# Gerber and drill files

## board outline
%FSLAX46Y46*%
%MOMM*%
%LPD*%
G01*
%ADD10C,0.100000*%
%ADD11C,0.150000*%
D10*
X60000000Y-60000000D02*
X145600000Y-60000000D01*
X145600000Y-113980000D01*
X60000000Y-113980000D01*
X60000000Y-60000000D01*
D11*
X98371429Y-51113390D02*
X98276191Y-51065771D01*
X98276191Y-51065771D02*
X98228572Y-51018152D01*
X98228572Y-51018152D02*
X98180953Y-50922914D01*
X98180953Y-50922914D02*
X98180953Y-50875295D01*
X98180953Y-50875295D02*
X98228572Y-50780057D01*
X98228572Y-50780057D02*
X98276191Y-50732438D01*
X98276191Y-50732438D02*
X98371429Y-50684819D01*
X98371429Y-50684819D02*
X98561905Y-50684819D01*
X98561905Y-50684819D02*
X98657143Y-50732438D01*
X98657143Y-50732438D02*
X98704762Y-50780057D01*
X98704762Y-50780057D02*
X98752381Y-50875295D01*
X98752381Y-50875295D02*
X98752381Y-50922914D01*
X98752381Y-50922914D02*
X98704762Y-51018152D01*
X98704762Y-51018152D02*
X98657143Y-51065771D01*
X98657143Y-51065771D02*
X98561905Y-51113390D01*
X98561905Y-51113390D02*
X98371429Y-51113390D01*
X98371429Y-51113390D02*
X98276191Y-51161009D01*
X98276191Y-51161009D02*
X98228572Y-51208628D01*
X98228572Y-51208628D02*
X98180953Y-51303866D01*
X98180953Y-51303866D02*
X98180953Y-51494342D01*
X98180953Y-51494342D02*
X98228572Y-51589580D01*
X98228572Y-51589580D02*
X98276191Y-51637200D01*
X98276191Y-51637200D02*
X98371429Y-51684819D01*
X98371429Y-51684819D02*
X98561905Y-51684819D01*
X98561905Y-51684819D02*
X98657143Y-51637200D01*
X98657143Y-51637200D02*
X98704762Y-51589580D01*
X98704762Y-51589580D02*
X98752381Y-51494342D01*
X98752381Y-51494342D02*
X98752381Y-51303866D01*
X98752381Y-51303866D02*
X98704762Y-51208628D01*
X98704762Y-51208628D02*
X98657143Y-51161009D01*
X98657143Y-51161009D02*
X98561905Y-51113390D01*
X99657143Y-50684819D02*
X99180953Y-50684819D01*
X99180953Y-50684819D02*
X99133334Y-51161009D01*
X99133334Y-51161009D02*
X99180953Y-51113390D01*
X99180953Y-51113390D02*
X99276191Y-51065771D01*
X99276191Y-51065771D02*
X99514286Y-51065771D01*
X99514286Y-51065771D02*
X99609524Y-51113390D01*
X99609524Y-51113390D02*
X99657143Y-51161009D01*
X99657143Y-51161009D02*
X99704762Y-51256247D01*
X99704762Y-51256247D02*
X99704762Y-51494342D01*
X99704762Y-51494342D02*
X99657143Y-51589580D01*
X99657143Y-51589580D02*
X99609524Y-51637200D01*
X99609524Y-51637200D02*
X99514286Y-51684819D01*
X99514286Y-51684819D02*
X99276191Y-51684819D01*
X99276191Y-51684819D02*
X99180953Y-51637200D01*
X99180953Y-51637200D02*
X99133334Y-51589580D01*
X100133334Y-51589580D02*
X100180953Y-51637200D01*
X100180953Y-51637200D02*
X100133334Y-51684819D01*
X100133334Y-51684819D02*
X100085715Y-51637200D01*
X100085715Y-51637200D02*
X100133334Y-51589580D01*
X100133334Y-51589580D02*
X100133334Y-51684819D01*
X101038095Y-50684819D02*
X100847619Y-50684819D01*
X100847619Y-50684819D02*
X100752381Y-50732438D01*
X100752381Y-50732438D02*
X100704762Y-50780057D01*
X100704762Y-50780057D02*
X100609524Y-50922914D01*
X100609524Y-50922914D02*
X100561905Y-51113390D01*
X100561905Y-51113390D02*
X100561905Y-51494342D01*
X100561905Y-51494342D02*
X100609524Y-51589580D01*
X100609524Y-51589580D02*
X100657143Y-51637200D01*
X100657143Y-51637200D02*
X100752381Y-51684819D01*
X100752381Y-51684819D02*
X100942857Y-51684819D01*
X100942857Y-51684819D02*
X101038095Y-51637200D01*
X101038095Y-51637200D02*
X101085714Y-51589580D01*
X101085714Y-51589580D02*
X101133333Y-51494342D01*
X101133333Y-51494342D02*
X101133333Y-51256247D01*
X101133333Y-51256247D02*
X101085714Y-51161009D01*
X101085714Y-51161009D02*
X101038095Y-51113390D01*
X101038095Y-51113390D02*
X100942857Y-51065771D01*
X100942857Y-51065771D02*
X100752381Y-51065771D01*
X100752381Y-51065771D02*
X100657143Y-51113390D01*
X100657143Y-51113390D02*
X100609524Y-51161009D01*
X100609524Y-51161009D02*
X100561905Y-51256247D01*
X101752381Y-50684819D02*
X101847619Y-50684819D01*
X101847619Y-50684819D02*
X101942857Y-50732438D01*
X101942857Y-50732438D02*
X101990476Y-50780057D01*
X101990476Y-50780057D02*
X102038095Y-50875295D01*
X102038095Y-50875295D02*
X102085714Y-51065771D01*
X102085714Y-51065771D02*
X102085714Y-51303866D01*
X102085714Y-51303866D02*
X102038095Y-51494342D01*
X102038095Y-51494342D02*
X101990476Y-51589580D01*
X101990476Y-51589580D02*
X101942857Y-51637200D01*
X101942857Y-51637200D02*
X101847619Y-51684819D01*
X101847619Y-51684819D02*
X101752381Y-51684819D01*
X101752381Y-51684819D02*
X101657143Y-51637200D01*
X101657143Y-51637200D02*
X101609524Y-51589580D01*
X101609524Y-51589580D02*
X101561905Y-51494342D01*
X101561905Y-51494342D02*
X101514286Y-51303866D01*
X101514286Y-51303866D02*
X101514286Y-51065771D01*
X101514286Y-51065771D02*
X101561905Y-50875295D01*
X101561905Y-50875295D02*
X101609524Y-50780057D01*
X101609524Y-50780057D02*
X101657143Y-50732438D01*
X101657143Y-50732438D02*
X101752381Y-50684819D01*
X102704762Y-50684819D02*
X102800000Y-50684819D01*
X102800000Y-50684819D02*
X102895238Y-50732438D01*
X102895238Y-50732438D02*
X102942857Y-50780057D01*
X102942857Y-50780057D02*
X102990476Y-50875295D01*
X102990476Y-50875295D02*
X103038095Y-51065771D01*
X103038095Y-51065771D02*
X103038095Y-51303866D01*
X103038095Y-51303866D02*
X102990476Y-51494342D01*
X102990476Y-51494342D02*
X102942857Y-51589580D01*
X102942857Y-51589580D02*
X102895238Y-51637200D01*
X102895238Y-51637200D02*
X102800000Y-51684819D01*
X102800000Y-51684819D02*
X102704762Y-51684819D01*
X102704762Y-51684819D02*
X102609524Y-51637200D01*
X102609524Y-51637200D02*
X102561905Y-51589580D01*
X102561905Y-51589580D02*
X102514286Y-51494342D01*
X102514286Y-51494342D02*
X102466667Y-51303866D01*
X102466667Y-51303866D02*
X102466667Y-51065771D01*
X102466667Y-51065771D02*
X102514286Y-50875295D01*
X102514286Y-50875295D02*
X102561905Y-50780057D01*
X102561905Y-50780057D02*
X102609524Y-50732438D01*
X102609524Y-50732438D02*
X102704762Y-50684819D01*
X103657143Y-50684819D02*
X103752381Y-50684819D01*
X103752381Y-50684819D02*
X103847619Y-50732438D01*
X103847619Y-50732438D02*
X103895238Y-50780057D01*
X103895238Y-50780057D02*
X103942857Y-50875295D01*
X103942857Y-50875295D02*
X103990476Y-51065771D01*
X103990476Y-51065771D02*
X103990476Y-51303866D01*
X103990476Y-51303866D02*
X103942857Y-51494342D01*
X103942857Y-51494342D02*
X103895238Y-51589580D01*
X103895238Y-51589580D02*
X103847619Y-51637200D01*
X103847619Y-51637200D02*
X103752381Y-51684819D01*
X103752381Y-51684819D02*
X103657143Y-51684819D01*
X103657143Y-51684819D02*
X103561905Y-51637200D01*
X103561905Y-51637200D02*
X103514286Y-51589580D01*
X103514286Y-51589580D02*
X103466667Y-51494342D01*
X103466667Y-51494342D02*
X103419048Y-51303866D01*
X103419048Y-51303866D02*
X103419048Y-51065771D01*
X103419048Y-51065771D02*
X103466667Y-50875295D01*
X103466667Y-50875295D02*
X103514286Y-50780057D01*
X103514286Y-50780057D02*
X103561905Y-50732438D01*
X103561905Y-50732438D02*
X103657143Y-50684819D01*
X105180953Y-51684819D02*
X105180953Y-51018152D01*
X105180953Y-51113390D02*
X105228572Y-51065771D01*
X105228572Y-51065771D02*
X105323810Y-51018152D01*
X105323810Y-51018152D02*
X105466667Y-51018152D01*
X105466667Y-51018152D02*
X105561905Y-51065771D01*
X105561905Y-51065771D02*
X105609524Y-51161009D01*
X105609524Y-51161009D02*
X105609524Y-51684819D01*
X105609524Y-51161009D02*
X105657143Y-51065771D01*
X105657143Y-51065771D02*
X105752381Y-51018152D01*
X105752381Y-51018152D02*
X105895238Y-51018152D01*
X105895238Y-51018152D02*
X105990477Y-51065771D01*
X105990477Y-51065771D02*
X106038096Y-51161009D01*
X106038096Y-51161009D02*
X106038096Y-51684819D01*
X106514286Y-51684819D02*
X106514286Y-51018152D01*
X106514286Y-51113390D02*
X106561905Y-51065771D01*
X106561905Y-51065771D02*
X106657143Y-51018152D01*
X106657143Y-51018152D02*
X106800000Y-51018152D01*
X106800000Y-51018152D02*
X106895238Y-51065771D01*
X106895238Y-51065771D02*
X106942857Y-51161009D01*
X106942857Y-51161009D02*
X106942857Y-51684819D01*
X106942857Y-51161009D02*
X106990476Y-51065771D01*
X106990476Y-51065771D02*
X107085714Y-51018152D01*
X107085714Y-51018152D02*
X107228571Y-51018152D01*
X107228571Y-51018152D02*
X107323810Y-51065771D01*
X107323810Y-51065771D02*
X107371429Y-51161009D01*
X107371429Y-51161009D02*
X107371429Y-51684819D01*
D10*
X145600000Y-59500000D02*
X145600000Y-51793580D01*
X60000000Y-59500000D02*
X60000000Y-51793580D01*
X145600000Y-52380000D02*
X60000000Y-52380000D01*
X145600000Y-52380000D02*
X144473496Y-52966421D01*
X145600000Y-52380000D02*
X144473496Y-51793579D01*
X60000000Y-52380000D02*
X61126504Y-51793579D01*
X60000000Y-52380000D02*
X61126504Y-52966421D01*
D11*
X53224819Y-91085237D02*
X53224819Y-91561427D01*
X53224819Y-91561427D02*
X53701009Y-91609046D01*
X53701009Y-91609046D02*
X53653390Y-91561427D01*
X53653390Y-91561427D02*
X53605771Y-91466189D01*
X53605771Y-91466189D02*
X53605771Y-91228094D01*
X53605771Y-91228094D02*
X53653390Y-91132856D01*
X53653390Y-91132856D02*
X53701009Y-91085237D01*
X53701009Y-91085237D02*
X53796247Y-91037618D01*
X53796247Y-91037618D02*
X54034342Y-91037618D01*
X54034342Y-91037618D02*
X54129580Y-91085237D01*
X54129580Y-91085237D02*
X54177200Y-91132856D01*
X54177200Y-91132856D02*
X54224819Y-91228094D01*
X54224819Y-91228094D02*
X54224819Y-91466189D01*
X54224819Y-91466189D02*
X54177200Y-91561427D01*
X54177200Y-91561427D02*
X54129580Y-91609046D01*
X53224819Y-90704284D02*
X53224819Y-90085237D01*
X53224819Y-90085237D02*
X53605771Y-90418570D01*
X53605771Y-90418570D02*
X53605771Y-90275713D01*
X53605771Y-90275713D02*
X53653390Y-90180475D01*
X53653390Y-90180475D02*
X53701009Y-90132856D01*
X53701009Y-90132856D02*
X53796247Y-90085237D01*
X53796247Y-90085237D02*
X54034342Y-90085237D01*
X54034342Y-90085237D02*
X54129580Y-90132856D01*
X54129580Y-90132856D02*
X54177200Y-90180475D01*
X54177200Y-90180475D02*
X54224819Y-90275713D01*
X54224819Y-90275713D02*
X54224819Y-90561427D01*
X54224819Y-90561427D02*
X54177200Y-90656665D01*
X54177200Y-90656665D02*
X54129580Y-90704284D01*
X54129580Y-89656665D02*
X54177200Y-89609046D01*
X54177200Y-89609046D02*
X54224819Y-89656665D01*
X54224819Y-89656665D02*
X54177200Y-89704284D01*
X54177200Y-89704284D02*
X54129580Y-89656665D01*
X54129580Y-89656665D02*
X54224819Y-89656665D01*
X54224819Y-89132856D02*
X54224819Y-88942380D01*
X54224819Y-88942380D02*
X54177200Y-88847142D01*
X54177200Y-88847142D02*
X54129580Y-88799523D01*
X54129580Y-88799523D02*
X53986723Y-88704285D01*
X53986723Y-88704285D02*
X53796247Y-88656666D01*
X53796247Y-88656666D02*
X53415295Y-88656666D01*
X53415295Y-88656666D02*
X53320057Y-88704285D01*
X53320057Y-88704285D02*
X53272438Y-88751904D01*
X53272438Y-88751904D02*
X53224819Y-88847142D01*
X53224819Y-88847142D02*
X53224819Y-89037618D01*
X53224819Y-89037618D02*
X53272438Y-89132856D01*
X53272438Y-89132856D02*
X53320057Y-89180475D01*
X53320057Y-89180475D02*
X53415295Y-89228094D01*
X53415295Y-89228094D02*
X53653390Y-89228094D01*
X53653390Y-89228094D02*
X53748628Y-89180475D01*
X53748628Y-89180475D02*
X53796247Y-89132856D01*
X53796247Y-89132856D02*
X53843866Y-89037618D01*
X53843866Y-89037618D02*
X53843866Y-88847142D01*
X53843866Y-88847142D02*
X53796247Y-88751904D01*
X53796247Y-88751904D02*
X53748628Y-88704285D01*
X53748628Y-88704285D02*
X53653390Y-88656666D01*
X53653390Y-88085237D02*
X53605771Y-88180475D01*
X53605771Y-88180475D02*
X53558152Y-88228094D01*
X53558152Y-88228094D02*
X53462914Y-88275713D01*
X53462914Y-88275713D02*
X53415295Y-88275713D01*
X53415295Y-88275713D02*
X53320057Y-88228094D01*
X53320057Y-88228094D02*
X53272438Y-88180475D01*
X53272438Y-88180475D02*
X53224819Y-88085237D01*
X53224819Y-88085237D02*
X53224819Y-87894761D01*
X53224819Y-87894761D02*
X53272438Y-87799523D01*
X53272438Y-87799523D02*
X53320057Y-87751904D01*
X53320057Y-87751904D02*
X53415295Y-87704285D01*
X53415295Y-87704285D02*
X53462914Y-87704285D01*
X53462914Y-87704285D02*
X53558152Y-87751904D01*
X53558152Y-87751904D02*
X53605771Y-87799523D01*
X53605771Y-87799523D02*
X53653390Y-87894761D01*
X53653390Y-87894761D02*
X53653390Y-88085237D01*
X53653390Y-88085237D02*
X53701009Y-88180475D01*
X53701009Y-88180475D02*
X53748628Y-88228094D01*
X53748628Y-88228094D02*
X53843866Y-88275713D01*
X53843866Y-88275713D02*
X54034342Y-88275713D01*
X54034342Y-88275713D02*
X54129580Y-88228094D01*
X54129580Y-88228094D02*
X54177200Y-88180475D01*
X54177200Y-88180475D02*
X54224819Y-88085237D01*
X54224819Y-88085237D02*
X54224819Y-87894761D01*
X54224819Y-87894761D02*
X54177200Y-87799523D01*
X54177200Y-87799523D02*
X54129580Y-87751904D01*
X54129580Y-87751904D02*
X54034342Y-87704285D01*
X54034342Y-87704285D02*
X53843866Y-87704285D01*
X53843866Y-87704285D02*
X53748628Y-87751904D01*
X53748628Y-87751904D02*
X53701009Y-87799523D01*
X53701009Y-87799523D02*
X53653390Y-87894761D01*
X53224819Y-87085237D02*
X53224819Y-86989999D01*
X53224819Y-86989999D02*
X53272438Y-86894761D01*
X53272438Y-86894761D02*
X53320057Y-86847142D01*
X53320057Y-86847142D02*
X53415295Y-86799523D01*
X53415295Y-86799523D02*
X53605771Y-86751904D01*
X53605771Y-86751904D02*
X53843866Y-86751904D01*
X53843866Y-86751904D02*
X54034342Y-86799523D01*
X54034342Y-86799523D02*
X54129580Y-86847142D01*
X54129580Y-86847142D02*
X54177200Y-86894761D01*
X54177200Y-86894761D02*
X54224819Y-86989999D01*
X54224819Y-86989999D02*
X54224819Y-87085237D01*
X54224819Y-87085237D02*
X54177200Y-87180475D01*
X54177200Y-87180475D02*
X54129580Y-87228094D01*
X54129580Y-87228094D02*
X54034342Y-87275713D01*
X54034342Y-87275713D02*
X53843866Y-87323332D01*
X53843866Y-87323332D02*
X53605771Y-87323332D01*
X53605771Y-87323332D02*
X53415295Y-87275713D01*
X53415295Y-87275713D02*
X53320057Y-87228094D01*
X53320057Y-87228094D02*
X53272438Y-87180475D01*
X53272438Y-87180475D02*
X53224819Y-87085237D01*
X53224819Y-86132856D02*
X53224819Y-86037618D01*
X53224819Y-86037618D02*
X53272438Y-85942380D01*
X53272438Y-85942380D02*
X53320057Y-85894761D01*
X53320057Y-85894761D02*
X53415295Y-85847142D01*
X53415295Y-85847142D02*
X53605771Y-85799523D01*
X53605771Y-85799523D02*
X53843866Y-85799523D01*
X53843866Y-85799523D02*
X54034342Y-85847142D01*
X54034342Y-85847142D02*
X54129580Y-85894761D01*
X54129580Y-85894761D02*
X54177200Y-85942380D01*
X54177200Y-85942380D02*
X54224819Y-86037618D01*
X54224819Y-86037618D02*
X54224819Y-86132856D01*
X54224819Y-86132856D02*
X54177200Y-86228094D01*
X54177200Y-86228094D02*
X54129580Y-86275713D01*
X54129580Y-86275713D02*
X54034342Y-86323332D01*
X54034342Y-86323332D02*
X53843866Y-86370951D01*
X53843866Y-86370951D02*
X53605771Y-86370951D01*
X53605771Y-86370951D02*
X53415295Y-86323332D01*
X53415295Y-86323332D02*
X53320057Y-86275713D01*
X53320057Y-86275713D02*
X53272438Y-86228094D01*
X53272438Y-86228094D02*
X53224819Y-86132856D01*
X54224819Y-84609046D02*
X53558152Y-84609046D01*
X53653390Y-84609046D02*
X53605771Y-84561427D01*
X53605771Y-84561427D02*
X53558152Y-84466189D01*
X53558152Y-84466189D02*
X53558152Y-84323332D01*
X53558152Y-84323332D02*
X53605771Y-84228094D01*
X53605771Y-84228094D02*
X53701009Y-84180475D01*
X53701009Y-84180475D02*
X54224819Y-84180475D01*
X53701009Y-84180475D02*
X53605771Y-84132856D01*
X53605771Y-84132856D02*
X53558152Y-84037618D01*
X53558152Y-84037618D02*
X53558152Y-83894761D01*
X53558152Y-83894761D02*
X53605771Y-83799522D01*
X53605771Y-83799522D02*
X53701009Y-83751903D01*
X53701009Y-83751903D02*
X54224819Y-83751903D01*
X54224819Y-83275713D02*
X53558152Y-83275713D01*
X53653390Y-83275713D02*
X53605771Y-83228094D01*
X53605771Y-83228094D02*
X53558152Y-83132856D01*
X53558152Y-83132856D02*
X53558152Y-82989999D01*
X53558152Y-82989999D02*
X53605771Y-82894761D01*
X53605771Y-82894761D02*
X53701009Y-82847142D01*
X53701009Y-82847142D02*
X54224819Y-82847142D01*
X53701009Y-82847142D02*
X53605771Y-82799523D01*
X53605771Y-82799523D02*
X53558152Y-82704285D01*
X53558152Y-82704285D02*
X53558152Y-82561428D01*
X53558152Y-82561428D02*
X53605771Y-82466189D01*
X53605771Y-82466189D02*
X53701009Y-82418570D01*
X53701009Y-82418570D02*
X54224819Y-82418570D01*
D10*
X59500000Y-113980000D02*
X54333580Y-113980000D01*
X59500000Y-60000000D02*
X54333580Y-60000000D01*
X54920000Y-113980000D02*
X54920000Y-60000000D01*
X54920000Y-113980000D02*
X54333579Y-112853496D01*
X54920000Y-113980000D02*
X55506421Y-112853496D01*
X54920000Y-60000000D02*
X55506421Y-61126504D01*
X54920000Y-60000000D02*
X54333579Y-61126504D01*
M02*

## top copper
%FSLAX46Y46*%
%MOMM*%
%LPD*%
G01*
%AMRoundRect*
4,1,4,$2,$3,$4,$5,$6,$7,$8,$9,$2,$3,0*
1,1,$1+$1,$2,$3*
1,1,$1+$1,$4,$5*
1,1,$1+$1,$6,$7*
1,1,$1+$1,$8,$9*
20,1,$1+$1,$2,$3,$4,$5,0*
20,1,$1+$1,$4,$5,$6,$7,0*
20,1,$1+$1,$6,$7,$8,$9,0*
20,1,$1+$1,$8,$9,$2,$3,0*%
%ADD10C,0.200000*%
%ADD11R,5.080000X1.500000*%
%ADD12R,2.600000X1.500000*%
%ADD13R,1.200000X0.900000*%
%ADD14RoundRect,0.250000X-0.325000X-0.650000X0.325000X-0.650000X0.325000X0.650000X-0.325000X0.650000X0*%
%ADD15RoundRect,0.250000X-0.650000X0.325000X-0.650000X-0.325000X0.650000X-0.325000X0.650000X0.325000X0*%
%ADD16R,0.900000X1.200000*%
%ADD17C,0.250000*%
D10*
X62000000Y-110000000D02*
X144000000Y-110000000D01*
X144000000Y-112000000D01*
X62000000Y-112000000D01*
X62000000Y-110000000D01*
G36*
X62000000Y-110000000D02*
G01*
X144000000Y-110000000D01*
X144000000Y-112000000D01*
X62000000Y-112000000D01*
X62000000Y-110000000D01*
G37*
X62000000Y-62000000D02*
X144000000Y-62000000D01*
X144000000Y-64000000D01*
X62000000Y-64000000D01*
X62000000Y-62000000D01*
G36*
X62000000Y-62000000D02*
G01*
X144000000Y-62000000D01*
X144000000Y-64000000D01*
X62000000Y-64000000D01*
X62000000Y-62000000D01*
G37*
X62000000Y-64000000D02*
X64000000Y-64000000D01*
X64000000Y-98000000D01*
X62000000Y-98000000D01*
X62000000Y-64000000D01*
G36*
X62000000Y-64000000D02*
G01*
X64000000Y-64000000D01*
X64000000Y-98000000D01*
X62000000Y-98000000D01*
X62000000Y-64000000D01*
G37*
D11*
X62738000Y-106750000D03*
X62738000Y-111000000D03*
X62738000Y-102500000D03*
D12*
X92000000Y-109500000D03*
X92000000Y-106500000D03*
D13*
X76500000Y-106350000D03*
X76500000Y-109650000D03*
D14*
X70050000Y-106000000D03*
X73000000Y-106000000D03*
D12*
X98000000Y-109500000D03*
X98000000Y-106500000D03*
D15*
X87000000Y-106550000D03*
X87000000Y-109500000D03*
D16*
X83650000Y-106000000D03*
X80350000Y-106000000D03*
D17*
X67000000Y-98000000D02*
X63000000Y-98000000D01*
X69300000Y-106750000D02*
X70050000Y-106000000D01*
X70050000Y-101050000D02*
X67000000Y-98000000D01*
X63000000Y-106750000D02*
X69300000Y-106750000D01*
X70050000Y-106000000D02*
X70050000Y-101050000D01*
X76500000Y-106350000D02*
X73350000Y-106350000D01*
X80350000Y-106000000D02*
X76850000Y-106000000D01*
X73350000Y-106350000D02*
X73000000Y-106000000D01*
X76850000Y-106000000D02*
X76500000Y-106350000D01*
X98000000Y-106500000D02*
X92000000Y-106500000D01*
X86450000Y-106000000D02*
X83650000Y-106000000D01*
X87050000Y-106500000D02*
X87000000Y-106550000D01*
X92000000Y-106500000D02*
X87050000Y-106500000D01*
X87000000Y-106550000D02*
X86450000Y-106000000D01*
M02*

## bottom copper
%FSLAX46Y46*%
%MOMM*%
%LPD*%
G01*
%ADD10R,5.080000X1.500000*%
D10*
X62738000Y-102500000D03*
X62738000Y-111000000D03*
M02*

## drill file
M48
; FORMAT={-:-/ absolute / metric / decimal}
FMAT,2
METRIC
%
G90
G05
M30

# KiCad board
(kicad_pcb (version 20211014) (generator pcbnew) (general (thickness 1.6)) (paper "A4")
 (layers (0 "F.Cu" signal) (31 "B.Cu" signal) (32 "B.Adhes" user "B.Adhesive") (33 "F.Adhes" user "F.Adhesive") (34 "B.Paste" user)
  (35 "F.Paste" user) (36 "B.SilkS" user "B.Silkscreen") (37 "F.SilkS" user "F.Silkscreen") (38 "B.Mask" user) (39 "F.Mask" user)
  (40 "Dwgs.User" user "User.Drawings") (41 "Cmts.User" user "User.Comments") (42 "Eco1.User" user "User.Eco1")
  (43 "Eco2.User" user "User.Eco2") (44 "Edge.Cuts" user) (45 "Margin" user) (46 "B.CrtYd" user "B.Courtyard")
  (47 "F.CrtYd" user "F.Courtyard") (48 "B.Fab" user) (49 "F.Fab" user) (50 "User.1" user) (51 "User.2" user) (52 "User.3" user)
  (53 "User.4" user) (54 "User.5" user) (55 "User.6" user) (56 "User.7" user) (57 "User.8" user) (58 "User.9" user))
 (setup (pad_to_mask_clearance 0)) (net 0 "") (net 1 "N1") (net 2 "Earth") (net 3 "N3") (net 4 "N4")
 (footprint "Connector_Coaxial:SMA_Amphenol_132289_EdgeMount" (layer "F.Cu") (at 62.738 106.75 180)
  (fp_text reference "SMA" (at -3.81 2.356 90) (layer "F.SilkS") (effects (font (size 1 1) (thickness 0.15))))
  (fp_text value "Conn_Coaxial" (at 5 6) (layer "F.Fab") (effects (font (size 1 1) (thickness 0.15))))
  (pad "1" smd rect (at 0 0 270) (size 1.5 5.08) (layers "F.Cu" "F.Paste" "F.Mask") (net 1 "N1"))
  (pad "2" smd rect (at 0 4.25 270) (size 1.5 5.08) (layers "B.Cu" "B.Paste" "B.Mask") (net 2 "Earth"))
  (pad "2" smd rect (at 0 -4.25 270) (size 1.5 5.08) (layers "F.Cu" "F.Paste" "F.Mask") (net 2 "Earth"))
  (pad "2" smd rect (at 0 4.25 270) (size 1.5 5.08) (layers "F.Cu" "F.Paste" "F.Mask") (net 2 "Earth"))
  (pad "2" smd rect (at 0 -4.25 270) (size 1.5 5.08) (layers "B.Cu" "B.Paste" "B.Mask") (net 2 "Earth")))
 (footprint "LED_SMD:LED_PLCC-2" (layer "F.Cu") (at 92 108 90)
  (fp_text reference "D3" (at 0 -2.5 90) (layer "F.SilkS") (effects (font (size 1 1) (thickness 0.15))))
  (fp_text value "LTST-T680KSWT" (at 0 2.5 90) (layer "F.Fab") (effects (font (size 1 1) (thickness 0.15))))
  (pad "1" smd rect (at -1.5 0 90) (size 1.5 2.6) (layers "F.Cu" "F.Paste" "F.Mask") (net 2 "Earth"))
  (pad "2" smd rect (at 1.5 0 90) (size 1.5 2.6) (layers "F.Cu" "F.Paste" "F.Mask") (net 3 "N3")))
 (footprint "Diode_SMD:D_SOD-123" (layer "F.Cu") (at 76.5 108 -90)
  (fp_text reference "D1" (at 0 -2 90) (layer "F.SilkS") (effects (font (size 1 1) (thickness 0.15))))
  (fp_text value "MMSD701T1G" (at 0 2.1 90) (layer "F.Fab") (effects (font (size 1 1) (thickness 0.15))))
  (pad "1" smd rect (at -1.65 0 270) (size 0.9 1.2) (layers "F.Cu" "F.Paste" "F.Mask") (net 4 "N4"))
  (pad "2" smd rect (at 1.65 0 270) (size 0.9 1.2) (layers "F.Cu" "F.Paste" "F.Mask") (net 2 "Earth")))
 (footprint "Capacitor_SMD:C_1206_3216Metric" (layer "F.Cu") (at 71.525 106)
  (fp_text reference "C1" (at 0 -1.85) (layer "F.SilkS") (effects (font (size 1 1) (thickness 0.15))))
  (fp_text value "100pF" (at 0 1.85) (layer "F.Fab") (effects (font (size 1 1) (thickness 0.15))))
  (pad "1" smd roundrect (at -1.475 0) (size 1.15 1.8) (layers "F.Cu" "F.Paste" "F.Mask") (roundrect_rratio 0.217391) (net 1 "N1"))
  (pad "2" smd roundrect (at 1.475 0) (size 1.15 1.8) (layers "F.Cu" "F.Paste" "F.Mask") (roundrect_rratio 0.217391) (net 4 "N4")))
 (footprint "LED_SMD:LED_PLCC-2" (layer "F.Cu") (at 98 108 90)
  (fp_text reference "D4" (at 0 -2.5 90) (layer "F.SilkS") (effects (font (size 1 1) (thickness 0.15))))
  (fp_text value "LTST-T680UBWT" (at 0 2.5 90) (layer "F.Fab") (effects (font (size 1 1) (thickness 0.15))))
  (pad "1" smd rect (at -1.5 0 90) (size 1.5 2.6) (layers "F.Cu" "F.Paste" "F.Mask") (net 2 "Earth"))
  (pad "2" smd rect (at 1.5 0 90) (size 1.5 2.6) (layers "F.Cu" "F.Paste" "F.Mask") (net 3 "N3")))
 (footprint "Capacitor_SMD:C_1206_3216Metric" (layer "F.Cu") (at 87 108.025 -90)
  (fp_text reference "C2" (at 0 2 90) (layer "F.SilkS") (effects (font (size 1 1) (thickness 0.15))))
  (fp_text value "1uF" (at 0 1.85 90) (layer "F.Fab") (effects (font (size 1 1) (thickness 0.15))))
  (pad "1" smd roundrect (at -1.475 0 270) (size 1.15 1.8) (layers "F.Cu" "F.Paste" "F.Mask") (roundrect_rratio 0.217391) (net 3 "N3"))
  (pad "2" smd roundrect (at 1.475 0 270) (size 1.15 1.8) (layers "F.Cu" "F.Paste" "F.Mask") (roundrect_rratio 0.217391) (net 2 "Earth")))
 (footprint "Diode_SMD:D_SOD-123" (layer "F.Cu") (at 82 106 180)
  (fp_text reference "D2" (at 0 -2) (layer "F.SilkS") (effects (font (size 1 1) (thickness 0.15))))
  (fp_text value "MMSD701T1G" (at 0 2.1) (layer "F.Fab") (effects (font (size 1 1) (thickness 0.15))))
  (pad "1" smd rect (at -1.65 0 180) (size 0.9 1.2) (layers "F.Cu" "F.Paste" "F.Mask") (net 3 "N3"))
  (pad "2" smd rect (at 1.65 0 180) (size 0.9 1.2) (layers "F.Cu" "F.Paste" "F.Mask") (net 4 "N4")))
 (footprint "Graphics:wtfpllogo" (layer "B.Cu") (at 140.5 64 180)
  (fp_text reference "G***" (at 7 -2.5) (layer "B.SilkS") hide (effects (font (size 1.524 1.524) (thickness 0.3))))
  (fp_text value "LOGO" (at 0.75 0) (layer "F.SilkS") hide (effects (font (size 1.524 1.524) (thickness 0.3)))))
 (gr_rect (start 62 112) (end 144 110) (layer "F.Cu") (width 0.2) (fill solid))
 (gr_rect (start 144 62) (end 62 64) (layer "F.Cu") (width 0.2) (fill solid))
 (gr_rect (start 62 64) (end 64 98) (layer "F.Cu") (width 0.2) (fill solid))
 (gr_rect (start 60 60) (end 145.6 113.98) (layer "Edge.Cuts") (width 0.1) (fill none))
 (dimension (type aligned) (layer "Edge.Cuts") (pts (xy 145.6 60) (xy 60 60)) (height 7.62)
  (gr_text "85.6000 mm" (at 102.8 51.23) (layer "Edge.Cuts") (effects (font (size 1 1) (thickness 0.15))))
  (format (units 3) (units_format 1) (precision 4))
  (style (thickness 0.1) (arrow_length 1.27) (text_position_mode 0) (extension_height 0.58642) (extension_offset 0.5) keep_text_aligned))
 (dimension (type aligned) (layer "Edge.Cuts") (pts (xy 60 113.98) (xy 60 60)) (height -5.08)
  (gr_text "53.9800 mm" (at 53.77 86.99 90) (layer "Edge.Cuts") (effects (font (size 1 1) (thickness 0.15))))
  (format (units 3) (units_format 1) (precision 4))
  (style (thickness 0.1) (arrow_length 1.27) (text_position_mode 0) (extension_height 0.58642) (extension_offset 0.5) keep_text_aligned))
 (segment (start 67 98) (end 63 98) (width 0.25) (layer "F.Cu") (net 1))
 (segment (start 69.3 106.75) (end 70.05 106) (width 0.25) (layer "F.Cu") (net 1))
 (segment (start 70.05 101.05) (end 67 98) (width 0.25) (layer "F.Cu") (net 1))
 (segment (start 63 106.75) (end 69.3 106.75) (width 0.25) (layer "F.Cu") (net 1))
 (segment (start 70.05 106) (end 70.05 101.05) (width 0.25) (layer "F.Cu") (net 1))
 (segment (start 76.5 106.35) (end 73.35 106.35) (width 0.25) (layer "F.Cu") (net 4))
 (segment (start 80.35 106) (end 76.85 106) (width 0.25) (layer "F.Cu") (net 4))
 (segment (start 73.35 106.35) (end 73 106) (width 0.25) (layer "F.Cu") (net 4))
 (segment (start 76.85 106) (end 76.5 106.35) (width 0.25) (layer "F.Cu") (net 4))
 (segment (start 98 106.5) (end 92 106.5) (width 0.25) (layer "F.Cu") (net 3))
 (segment (start 86.45 106) (end 83.65 106) (width 0.25) (layer "F.Cu") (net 3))
 (segment (start 87.05 106.5) (end 87 106.55) (width 0.25) (layer "F.Cu") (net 3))
 (segment (start 92 106.5) (end 87.05 106.5) (width 0.25) (layer "F.Cu") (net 3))
 (segment (start 87 106.55) (end 86.45 106) (width 0.25) (layer "F.Cu") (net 3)))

